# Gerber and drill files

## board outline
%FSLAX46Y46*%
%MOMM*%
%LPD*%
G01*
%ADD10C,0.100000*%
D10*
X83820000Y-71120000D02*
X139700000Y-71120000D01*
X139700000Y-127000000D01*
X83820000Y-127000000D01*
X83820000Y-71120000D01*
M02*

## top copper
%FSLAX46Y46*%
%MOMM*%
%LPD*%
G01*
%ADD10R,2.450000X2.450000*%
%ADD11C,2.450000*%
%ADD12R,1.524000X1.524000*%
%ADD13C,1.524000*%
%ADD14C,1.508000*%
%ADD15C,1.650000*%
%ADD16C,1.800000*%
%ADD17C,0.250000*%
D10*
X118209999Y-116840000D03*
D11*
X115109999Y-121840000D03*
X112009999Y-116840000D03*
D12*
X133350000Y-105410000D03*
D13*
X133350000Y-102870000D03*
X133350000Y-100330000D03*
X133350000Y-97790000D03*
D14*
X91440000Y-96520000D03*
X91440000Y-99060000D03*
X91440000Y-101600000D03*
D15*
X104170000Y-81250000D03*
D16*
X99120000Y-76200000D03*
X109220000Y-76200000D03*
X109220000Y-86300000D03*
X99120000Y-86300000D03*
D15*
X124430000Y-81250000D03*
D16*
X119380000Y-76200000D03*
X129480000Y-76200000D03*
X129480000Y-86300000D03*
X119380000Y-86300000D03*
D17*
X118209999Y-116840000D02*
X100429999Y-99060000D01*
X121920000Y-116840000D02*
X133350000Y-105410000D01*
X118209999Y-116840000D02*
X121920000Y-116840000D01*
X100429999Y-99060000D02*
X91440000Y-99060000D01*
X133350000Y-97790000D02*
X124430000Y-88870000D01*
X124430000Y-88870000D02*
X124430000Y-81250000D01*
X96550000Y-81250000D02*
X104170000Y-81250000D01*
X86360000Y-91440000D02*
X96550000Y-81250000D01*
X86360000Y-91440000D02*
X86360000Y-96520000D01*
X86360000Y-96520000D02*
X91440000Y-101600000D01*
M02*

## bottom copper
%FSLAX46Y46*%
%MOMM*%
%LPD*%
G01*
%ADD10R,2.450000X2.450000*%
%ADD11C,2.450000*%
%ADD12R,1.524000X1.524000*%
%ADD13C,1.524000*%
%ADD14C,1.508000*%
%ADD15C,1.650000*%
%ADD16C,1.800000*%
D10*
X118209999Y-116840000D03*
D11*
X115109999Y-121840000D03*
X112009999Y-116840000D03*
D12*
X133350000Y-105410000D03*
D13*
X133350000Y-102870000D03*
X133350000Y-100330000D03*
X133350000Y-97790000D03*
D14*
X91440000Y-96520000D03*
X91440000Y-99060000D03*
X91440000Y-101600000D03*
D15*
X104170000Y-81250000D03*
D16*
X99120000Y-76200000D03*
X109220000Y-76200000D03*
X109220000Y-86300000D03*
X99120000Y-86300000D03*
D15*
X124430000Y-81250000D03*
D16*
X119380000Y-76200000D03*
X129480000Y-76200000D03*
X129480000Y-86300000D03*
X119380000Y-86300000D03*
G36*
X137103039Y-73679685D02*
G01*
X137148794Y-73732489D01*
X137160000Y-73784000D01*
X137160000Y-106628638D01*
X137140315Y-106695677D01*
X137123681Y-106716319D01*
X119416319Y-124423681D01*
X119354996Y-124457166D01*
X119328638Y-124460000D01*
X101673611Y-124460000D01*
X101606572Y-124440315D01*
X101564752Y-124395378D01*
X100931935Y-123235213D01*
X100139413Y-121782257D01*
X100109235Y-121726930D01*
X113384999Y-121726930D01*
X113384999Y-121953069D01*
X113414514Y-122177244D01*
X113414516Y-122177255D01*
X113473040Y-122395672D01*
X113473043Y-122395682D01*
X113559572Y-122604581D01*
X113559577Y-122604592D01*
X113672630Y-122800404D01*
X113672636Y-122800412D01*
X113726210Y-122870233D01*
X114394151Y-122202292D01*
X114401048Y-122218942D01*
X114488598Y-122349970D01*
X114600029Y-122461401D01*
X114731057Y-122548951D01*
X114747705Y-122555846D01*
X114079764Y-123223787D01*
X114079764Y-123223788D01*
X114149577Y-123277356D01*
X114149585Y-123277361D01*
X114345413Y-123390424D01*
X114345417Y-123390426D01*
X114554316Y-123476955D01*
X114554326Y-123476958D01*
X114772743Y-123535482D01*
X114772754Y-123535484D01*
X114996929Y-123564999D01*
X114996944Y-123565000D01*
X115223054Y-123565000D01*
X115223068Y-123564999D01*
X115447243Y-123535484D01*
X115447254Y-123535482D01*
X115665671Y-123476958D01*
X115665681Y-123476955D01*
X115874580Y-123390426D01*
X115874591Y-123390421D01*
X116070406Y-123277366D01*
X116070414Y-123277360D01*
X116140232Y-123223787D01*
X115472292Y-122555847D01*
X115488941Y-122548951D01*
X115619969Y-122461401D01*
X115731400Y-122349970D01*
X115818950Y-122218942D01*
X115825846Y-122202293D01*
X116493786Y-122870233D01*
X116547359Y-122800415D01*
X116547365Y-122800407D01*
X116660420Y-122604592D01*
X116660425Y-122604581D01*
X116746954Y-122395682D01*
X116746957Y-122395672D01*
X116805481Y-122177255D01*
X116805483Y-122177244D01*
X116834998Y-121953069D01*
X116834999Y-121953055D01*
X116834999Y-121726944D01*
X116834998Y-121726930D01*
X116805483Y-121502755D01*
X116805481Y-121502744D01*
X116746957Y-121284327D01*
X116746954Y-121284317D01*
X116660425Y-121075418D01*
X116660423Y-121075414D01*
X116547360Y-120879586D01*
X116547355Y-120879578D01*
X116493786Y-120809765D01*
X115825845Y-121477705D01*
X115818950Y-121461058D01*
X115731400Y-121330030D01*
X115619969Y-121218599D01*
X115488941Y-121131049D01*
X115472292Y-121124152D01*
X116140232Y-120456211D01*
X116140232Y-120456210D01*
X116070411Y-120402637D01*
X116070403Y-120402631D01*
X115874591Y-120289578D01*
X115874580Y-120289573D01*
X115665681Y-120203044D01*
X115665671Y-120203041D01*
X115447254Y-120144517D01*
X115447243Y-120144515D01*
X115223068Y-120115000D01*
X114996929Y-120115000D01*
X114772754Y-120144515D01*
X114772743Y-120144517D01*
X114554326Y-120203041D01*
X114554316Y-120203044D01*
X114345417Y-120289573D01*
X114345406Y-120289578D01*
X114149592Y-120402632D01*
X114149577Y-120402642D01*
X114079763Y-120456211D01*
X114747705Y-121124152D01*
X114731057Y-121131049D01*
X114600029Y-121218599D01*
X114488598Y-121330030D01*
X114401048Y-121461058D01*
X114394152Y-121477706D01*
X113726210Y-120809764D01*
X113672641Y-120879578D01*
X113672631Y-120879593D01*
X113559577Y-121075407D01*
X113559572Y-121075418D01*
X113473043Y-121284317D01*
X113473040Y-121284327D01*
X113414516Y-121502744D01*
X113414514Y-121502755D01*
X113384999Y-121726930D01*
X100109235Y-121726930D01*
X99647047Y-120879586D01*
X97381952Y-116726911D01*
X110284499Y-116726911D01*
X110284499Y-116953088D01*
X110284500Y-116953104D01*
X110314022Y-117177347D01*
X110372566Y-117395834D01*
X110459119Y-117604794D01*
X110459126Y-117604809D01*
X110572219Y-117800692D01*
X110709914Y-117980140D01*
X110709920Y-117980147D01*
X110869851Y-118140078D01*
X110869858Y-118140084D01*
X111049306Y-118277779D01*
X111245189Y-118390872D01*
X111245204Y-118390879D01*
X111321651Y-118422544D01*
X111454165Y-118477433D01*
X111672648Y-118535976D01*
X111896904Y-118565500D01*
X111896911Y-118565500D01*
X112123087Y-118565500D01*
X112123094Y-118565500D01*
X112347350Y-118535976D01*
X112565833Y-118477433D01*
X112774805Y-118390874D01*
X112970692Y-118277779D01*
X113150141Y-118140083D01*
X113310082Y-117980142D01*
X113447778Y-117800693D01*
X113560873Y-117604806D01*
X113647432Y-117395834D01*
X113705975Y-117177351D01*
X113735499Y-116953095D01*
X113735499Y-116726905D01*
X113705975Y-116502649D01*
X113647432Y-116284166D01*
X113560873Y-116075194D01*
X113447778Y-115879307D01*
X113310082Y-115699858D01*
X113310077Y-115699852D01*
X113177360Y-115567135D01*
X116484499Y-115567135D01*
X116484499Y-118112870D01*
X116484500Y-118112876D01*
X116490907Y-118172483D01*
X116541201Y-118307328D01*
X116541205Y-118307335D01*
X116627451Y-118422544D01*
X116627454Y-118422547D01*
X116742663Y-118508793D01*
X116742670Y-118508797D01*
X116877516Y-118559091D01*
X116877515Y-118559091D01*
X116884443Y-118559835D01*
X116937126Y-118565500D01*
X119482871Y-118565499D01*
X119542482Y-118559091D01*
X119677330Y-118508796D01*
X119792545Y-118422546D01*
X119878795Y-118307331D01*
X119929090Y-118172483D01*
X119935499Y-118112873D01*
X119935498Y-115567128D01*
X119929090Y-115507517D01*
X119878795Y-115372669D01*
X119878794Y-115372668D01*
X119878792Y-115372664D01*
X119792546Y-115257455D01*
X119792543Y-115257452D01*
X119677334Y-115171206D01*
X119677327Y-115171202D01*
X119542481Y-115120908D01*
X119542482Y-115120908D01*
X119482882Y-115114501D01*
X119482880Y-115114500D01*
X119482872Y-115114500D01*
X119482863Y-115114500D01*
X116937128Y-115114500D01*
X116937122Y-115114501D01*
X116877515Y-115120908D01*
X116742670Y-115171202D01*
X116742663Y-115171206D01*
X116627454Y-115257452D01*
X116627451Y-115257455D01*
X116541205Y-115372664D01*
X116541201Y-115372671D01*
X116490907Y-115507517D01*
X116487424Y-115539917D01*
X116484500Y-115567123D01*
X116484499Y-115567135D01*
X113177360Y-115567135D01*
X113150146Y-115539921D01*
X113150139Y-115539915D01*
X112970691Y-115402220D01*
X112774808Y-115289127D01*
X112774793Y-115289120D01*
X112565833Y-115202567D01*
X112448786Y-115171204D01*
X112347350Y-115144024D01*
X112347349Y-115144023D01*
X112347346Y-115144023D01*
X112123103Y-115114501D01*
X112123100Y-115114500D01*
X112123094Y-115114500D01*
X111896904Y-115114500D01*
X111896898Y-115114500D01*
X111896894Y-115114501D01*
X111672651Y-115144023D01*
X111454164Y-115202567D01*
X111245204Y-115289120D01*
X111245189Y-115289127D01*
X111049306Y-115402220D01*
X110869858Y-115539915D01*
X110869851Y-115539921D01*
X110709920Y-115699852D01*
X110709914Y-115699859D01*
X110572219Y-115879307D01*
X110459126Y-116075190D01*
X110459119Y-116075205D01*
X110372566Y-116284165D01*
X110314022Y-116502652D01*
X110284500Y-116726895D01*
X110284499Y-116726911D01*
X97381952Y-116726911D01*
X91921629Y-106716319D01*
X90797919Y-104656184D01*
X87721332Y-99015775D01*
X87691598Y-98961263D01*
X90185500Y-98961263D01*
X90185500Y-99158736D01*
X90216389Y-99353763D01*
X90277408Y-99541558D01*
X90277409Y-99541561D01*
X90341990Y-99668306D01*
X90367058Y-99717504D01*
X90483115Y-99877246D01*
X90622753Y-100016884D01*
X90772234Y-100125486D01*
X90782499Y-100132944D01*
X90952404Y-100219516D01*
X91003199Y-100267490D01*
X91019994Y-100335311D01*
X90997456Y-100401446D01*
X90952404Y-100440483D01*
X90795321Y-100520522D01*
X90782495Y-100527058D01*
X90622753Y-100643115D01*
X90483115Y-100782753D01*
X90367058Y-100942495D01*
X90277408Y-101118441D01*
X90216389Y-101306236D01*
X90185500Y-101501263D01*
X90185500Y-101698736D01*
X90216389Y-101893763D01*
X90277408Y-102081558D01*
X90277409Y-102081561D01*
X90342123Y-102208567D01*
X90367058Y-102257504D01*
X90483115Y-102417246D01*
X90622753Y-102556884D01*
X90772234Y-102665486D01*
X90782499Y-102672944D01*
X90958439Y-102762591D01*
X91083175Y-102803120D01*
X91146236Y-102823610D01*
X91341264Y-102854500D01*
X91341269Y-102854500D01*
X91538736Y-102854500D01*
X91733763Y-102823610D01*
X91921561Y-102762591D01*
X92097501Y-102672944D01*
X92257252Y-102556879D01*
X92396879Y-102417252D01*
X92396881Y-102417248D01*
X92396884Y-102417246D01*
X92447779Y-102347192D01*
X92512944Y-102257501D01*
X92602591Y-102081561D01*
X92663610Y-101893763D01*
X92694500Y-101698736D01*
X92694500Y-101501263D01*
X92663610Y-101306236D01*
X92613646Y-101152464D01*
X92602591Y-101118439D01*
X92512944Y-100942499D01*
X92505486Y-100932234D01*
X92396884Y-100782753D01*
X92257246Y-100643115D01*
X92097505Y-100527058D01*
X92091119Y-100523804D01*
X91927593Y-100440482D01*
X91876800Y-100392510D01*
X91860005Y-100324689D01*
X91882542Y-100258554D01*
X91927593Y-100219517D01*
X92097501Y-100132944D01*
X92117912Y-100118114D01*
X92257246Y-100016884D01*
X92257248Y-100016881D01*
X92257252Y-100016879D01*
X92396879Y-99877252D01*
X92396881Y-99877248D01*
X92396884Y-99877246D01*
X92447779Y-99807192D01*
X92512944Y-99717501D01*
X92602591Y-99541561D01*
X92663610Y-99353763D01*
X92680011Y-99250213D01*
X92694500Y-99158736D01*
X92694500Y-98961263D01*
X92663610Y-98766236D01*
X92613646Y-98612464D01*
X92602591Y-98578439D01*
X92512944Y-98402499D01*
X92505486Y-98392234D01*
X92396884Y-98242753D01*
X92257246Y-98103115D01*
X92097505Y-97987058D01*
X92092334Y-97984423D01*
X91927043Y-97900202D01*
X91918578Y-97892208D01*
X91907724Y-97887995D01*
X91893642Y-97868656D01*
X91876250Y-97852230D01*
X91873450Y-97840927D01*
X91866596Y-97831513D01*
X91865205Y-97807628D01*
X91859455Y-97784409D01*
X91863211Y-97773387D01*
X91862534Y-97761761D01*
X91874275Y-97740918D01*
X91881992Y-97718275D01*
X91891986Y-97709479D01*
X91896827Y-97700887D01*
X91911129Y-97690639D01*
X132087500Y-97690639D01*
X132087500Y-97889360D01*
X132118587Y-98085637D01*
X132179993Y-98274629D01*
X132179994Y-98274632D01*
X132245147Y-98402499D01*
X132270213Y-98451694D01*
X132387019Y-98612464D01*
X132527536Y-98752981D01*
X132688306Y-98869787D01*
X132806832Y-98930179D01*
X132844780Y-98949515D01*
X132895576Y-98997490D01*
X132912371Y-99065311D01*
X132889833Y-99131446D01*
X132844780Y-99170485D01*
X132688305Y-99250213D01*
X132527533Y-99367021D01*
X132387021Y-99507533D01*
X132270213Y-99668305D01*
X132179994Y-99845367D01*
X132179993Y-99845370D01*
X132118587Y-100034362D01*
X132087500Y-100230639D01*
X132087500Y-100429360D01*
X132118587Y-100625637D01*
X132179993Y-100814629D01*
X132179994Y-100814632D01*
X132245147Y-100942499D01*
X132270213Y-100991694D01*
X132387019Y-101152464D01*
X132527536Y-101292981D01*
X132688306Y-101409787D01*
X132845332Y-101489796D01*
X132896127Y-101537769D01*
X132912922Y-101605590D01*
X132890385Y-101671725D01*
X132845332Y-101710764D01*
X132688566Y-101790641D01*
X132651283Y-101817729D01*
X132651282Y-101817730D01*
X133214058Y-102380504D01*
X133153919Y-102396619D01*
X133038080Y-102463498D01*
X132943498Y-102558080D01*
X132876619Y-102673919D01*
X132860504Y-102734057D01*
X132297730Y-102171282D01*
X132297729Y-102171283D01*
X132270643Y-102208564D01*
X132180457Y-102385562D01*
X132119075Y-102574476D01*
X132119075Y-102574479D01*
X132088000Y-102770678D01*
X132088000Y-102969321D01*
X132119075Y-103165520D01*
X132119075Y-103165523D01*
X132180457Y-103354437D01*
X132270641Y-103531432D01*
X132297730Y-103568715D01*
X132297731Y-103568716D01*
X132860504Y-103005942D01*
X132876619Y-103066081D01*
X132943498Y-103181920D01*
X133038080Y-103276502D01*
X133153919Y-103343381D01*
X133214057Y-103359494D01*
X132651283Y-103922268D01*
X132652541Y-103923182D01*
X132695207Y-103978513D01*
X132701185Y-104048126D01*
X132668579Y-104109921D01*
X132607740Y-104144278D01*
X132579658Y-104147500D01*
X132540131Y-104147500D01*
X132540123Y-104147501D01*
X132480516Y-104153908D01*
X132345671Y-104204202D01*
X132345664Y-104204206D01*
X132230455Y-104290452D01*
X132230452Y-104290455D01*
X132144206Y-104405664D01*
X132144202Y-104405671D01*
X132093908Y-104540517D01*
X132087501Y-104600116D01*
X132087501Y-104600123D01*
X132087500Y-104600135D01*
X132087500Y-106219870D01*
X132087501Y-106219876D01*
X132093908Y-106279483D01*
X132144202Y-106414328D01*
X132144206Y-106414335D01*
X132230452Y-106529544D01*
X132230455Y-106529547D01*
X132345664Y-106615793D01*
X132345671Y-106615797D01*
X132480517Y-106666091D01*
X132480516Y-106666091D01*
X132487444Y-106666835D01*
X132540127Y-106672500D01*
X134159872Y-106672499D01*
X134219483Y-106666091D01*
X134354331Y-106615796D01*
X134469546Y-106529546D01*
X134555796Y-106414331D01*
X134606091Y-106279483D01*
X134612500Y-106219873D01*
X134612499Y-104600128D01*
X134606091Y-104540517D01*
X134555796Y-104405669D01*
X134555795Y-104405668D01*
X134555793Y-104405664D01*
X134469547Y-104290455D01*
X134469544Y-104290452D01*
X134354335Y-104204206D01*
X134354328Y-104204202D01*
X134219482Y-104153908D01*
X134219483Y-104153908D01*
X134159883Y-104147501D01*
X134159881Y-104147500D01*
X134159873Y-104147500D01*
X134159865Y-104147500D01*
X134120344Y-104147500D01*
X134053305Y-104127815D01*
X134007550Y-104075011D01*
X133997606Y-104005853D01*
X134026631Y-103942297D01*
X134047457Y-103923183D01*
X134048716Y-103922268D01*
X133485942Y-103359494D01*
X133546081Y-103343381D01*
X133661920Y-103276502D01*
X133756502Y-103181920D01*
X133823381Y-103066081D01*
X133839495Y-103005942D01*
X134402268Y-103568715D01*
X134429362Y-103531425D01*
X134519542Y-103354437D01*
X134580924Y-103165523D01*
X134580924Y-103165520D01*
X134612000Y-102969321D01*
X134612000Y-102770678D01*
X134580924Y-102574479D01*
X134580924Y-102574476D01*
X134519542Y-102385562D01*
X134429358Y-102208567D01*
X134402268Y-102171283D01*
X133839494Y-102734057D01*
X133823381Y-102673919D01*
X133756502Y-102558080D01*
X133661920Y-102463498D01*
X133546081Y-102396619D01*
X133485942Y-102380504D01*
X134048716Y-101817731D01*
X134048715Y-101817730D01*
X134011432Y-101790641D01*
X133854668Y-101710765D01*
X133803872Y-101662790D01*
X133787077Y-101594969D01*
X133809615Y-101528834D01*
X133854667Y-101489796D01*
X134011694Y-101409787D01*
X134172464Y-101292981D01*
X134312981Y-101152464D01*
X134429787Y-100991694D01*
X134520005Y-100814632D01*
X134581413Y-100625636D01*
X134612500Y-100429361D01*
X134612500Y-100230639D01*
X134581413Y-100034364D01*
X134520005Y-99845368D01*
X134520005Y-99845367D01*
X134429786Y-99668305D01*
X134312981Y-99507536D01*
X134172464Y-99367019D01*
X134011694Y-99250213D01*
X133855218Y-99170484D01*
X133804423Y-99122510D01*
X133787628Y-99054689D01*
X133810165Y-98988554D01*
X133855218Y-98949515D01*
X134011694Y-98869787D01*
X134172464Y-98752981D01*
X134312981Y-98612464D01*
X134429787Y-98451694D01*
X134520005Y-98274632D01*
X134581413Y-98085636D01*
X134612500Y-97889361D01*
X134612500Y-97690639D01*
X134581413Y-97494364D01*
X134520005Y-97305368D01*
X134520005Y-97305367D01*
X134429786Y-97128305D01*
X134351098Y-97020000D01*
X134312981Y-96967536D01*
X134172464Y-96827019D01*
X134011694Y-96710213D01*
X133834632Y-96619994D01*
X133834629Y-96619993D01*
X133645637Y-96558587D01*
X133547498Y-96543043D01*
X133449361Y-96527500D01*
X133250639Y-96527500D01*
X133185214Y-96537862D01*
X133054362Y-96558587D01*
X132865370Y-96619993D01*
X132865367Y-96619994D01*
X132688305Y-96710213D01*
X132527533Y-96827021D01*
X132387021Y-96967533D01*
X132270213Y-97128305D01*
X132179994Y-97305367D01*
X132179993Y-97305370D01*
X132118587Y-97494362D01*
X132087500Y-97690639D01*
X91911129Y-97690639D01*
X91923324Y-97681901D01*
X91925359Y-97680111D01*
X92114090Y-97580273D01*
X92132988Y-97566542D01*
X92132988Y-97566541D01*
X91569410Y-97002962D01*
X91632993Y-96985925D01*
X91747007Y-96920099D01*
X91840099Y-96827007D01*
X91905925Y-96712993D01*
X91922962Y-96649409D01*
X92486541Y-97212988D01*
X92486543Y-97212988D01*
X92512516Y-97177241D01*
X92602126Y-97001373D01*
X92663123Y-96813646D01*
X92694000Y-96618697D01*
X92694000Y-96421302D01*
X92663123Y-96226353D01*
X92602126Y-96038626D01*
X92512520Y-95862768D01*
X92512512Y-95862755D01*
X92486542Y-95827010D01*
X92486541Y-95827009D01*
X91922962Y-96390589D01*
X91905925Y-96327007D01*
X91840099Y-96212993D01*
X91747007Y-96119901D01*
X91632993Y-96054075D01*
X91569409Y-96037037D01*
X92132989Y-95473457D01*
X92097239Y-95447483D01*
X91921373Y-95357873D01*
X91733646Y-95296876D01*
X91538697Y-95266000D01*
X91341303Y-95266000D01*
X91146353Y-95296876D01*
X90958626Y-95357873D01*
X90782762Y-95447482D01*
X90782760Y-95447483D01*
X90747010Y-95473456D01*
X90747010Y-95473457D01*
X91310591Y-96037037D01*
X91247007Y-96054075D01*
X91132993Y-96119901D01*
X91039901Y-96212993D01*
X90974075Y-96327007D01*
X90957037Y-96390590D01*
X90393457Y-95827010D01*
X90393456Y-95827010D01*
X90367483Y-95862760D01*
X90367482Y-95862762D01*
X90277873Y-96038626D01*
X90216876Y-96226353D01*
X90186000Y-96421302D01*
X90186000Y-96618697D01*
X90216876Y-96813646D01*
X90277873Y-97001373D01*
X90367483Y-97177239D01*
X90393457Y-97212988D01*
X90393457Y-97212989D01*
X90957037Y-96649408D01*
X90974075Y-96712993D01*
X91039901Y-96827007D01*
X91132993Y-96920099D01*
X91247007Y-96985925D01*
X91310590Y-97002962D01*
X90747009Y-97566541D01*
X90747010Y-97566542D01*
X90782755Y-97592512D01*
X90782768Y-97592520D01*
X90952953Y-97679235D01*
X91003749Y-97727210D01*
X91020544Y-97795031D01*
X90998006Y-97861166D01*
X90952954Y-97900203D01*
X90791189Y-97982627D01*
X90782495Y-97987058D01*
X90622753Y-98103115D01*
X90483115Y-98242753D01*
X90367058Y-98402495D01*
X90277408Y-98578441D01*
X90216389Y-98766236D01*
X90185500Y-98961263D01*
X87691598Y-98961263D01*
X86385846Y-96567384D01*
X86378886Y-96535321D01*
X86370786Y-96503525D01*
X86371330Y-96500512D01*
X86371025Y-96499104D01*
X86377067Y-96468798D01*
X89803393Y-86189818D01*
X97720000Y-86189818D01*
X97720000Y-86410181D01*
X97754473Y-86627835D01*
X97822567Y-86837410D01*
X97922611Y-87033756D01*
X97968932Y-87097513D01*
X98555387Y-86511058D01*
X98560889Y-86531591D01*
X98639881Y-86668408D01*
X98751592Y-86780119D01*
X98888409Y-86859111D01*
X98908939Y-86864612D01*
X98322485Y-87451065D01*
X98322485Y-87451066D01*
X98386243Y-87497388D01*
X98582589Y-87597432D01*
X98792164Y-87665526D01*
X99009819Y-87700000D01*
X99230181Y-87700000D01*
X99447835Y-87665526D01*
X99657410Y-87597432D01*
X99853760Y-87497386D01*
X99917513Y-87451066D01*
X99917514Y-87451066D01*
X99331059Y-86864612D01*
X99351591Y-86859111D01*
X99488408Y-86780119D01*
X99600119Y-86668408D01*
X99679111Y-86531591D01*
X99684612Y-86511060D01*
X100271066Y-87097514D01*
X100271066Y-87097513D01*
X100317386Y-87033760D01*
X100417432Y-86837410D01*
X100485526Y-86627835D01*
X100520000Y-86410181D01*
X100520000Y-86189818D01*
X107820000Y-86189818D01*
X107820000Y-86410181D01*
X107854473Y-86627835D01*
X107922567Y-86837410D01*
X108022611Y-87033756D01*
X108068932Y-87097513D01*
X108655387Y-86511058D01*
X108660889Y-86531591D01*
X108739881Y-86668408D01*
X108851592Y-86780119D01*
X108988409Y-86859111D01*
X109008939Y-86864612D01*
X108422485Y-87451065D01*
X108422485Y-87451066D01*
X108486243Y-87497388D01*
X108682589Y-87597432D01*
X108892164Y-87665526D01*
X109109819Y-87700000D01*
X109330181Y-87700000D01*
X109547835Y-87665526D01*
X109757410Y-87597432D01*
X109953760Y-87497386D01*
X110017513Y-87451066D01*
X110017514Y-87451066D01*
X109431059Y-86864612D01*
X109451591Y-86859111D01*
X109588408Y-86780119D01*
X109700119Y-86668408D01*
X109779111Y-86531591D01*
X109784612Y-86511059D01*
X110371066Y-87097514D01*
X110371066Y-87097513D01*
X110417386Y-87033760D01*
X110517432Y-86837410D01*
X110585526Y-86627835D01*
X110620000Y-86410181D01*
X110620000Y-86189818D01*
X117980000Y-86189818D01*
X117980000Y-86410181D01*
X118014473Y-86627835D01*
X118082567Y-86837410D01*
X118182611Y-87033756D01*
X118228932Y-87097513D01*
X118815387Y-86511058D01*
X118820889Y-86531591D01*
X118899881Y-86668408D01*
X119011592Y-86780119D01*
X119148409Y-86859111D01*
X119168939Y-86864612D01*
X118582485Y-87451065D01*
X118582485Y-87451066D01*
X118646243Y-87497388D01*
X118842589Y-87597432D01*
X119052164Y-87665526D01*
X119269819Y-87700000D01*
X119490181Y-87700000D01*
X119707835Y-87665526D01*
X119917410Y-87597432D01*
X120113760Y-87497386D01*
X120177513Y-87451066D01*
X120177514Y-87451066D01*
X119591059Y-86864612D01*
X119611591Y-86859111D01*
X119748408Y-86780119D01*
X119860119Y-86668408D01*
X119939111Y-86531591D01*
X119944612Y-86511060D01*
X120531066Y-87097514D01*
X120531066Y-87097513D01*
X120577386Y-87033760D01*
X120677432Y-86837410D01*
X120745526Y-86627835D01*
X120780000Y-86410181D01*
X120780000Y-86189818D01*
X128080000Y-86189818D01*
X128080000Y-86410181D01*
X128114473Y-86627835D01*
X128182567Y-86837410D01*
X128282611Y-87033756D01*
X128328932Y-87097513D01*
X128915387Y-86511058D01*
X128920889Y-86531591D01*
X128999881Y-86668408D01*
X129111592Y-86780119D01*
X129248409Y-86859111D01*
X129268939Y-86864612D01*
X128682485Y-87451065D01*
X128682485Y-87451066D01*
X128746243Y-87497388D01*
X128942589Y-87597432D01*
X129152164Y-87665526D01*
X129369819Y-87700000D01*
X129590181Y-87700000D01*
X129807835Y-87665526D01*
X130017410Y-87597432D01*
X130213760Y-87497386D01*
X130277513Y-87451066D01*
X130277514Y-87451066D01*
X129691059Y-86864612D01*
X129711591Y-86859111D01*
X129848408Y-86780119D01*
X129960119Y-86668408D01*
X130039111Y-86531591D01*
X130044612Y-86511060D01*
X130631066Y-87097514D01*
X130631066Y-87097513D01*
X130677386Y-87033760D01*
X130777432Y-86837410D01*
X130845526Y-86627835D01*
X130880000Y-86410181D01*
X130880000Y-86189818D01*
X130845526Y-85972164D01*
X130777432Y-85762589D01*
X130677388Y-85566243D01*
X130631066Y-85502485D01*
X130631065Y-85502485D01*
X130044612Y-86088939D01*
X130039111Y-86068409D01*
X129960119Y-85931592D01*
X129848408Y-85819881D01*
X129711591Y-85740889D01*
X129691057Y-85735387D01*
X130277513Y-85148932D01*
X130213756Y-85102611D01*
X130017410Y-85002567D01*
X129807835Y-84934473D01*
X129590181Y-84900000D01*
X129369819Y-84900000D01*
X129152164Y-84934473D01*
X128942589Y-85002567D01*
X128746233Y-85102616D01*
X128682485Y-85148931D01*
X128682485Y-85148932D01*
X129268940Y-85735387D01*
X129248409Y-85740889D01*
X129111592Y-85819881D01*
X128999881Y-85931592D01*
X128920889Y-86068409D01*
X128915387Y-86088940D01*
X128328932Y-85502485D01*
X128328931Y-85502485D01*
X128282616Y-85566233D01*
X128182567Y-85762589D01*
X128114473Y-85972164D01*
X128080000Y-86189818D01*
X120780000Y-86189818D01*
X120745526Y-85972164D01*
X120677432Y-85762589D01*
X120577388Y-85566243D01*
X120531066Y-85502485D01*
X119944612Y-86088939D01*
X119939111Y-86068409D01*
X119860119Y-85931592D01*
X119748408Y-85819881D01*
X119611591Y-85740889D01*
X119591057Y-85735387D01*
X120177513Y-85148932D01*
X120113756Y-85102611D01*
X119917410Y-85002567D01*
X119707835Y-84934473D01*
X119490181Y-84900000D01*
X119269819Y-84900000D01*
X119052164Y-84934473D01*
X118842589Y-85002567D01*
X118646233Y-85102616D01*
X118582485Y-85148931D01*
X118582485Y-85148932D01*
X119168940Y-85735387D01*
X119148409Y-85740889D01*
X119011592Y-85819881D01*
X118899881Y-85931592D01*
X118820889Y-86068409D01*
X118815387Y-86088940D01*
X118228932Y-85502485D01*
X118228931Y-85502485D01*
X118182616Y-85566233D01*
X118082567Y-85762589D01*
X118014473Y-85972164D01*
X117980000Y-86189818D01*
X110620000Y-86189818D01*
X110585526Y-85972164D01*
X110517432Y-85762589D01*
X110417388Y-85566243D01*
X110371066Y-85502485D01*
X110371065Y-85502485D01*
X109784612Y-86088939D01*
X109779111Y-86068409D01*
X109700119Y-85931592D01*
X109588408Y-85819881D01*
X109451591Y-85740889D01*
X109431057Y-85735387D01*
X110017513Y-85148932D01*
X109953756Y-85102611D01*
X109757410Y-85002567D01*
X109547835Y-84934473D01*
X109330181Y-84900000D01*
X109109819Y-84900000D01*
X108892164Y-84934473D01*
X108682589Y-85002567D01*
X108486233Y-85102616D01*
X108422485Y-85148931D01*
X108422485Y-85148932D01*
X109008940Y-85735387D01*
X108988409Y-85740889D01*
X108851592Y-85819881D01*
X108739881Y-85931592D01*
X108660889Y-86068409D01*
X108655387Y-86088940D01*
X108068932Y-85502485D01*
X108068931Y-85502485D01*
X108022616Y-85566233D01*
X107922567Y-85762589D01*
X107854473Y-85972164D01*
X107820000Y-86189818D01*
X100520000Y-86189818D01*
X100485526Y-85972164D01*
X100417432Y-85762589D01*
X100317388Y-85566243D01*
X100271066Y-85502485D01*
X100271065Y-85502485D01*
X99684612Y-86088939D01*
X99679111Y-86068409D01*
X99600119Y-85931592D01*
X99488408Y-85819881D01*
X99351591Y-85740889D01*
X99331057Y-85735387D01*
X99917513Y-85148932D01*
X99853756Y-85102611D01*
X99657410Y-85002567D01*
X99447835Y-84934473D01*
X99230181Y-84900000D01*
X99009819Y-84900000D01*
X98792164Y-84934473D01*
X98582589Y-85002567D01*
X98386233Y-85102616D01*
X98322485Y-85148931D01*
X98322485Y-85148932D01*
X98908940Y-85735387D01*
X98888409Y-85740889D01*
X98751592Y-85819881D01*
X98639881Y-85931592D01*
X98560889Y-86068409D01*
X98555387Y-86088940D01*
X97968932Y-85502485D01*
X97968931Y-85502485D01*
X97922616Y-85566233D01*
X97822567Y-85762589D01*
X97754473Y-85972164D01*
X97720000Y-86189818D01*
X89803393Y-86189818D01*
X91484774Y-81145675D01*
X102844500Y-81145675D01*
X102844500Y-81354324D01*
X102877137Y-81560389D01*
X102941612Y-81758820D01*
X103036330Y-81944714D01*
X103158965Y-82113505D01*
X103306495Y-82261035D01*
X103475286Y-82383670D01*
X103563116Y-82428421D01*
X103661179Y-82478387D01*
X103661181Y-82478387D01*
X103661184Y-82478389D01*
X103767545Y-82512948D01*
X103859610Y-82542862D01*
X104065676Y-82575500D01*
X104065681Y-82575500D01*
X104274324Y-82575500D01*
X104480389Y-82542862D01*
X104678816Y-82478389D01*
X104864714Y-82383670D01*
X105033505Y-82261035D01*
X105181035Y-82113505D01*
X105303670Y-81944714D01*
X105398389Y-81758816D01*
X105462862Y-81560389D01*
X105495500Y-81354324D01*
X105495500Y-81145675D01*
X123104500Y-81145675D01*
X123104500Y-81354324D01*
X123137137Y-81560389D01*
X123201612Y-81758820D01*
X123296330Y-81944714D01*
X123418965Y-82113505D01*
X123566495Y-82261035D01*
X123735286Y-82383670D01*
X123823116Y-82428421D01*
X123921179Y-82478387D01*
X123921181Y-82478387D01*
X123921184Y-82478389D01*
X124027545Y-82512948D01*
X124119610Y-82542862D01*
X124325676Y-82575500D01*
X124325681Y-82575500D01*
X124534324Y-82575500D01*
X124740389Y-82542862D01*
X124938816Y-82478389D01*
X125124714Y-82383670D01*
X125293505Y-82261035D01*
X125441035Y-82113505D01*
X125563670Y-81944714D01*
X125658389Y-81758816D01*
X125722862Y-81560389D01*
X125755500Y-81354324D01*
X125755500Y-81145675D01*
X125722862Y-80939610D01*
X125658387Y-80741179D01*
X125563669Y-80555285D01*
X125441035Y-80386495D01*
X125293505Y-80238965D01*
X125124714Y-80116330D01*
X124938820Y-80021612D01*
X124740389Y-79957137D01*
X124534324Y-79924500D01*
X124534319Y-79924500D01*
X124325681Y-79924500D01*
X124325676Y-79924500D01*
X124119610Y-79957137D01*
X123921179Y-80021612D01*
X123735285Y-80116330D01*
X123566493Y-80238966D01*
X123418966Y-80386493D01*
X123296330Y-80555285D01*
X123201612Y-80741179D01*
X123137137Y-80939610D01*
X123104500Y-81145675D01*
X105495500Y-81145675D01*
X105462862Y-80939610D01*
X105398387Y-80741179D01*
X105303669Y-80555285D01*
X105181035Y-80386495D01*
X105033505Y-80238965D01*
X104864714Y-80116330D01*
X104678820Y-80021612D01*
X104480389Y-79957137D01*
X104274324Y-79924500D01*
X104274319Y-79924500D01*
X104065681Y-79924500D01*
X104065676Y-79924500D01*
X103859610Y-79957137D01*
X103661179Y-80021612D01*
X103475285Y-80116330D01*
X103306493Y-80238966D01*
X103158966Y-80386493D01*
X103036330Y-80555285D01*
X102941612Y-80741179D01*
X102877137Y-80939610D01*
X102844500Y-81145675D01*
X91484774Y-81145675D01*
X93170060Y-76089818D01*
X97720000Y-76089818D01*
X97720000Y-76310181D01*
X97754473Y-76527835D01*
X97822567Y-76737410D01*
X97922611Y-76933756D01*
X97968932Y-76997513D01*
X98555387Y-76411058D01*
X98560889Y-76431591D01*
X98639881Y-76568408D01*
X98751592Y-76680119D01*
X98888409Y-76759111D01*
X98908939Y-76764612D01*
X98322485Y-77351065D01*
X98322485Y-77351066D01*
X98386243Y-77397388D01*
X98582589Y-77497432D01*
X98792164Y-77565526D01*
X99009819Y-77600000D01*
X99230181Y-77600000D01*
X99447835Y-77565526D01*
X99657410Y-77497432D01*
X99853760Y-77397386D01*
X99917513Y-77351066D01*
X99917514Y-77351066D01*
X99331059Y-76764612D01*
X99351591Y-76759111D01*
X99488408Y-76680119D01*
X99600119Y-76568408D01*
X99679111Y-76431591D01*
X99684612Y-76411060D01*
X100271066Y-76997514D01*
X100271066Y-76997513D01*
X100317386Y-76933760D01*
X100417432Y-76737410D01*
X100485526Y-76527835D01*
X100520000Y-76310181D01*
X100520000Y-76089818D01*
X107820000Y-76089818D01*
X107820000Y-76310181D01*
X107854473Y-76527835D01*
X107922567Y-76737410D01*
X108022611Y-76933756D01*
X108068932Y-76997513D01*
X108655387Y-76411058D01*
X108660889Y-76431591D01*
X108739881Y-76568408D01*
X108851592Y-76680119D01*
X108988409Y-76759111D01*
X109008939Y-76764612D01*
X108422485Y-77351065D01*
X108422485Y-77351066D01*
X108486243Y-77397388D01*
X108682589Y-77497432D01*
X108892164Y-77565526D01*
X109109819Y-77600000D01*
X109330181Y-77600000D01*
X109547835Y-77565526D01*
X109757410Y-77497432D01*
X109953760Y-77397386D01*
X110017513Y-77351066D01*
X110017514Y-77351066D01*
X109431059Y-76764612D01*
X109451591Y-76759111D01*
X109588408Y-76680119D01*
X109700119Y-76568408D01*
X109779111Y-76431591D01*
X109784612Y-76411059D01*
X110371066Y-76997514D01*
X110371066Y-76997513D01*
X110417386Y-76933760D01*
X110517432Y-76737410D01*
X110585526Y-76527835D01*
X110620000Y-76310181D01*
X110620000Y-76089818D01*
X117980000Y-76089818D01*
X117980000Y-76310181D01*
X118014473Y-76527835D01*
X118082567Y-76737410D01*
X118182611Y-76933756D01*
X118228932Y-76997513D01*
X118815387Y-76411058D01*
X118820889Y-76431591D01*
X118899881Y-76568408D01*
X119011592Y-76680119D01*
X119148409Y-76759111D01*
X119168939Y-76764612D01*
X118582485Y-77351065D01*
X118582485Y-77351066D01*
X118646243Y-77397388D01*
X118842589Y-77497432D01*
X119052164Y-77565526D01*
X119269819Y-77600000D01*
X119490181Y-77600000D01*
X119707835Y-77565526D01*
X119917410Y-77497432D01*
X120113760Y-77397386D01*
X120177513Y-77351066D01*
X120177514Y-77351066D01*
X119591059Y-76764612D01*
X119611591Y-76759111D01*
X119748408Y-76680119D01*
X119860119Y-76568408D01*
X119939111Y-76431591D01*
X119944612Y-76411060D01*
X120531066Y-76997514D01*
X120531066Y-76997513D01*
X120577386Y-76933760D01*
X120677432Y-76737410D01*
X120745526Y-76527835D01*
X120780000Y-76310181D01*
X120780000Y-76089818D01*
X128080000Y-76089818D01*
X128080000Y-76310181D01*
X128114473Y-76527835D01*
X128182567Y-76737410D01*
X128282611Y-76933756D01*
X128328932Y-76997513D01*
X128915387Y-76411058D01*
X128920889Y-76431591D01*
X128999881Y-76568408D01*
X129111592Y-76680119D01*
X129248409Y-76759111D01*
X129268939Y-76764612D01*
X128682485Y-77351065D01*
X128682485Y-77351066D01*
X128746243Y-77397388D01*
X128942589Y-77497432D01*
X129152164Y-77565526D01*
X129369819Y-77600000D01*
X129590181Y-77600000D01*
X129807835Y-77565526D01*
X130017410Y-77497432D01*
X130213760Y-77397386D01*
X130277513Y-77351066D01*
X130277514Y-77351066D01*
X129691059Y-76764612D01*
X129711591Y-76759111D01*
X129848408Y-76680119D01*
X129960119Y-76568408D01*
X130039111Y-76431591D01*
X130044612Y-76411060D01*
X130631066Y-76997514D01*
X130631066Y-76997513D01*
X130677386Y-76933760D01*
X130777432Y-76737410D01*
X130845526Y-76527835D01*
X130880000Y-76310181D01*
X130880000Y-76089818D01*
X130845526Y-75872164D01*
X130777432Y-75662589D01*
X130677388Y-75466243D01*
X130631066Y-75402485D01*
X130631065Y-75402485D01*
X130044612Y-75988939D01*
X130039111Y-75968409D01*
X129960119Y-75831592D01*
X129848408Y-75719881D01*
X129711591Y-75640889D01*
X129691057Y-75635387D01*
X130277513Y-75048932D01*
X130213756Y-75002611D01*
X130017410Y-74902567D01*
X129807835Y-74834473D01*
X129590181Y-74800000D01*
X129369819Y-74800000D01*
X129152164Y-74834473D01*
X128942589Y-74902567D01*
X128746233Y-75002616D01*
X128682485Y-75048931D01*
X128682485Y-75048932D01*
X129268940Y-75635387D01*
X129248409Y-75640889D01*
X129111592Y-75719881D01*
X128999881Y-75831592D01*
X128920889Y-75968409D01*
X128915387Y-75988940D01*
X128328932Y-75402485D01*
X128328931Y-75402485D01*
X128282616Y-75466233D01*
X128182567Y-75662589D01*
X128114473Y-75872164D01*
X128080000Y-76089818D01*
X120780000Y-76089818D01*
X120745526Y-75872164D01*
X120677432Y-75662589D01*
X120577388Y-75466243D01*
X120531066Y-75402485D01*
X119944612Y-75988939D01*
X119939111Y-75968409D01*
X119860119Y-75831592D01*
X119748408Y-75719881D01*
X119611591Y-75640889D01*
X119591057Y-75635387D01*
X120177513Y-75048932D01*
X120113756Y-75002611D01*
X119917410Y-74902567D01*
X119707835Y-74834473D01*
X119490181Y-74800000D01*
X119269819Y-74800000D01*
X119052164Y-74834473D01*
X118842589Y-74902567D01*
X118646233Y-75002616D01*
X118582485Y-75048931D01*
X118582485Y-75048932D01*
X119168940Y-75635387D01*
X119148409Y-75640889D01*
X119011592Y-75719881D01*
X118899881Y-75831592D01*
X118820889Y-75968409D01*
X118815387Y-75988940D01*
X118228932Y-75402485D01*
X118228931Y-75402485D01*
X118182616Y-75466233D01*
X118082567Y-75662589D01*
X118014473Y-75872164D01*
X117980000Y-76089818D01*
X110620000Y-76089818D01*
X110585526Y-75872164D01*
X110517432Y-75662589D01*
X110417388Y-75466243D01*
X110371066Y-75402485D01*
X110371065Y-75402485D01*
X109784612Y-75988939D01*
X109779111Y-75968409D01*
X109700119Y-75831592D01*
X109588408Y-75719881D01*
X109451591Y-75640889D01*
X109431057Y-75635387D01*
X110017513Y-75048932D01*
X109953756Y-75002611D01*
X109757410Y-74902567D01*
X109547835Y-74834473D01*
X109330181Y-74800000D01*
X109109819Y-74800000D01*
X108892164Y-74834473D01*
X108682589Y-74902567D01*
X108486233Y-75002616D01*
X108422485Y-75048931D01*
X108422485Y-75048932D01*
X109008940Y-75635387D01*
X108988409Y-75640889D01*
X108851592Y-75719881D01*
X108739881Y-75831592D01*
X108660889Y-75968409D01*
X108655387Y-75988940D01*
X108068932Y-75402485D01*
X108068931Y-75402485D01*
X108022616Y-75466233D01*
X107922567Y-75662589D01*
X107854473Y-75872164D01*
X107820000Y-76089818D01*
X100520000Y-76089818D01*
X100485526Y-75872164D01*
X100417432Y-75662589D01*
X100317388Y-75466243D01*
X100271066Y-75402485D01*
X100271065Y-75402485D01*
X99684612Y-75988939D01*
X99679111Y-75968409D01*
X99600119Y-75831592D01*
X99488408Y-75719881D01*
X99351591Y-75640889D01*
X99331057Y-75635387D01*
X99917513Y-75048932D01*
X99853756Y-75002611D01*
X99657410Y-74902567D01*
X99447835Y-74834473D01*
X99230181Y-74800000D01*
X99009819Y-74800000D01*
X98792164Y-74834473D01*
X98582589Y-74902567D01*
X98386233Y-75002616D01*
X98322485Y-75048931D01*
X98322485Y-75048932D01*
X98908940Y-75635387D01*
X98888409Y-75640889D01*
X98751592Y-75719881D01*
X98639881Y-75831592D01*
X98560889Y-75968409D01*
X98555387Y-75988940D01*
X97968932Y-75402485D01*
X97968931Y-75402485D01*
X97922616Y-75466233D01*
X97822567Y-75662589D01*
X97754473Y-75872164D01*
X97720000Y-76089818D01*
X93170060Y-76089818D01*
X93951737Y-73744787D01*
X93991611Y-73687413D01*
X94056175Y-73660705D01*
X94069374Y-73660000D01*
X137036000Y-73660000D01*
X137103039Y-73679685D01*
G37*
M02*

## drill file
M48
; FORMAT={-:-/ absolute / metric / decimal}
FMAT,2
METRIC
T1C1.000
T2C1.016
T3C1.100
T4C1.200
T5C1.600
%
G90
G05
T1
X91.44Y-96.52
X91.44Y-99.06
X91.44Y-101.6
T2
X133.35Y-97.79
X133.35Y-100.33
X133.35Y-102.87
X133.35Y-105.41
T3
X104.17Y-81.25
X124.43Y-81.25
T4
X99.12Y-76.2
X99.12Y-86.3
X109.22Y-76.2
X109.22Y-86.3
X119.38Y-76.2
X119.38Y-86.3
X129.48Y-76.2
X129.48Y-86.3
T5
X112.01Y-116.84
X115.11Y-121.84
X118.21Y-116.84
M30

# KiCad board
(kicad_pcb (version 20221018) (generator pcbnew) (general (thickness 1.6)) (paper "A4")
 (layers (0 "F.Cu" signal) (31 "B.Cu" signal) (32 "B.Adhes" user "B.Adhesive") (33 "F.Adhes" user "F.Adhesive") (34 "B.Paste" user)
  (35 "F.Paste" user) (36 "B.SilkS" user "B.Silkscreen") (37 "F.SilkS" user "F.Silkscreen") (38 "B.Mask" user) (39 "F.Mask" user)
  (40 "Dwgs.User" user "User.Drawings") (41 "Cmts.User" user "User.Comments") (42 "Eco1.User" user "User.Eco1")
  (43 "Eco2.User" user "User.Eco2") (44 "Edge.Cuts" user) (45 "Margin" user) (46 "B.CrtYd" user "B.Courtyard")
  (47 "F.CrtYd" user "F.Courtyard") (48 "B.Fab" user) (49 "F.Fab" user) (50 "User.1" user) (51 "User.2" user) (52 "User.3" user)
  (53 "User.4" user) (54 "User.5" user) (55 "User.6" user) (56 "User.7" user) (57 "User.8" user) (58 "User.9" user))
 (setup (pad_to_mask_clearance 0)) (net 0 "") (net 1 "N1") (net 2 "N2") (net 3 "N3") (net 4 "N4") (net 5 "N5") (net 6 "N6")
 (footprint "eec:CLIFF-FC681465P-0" (layer "F.Cu") (at 111.76 116.84)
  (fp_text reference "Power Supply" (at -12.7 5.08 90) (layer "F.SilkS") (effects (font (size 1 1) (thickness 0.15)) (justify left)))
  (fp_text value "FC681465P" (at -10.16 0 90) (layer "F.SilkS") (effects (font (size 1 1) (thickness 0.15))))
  (pad "1" thru_hole rect (at 6.449999 0) (size 2.45 2.45) (drill 1.6) (layers "*.Cu") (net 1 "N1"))
  (pad "2" thru_hole circle (at 3.349999 5) (size 2.45 2.45) (drill 1.6) (layers "*.Cu") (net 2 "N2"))
  (pad "3" thru_hole circle (at 0.249999 0) (size 2.45 2.45) (drill 1.6) (layers "*.Cu") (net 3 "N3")))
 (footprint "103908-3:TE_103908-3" (layer "F.Cu") (at 133.35 101.6 90)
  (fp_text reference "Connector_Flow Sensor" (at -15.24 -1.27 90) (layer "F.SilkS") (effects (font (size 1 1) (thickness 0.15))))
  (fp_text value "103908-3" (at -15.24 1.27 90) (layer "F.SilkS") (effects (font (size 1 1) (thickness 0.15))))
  (pad "1" thru_hole rect (at -3.81 0 90) (size 1.524 1.524) (drill 1.016) (layers "*.Cu" "*.Mask") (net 1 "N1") (solder_mask_margin 0.102))
  (pad "2" thru_hole circle (at -1.27 0 90) (size 1.524 1.524) (drill 1.016) (layers "*.Cu" "*.Mask") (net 2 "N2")
   (solder_mask_margin 0.102))
  (pad "3" thru_hole circle (at 1.27 0 90) (size 1.524 1.524) (drill 1.016) (layers "*.Cu" "*.Mask") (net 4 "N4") (solder_mask_margin 0.102))
  (pad "4" thru_hole circle (at 3.81 0 90) (size 1.524 1.524) (drill 1.016) (layers "*.Cu" "*.Mask") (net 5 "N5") (solder_mask_margin 0.102)))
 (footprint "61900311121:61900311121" (layer "F.Cu") (at 91.44 99.06 90)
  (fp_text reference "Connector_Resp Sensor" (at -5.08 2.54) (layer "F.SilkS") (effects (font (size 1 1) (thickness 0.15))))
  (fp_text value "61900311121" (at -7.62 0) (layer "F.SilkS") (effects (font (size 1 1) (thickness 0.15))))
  (pad "1" thru_hole circle (at 2.54 0 90) (size 1.508 1.508) (drill 1) (layers "*.Cu" "*.Mask") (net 2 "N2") (solder_mask_margin 0.102))
  (pad "2" thru_hole circle (at 0 0 90) (size 1.508 1.508) (drill 1) (layers "*.Cu" "*.Mask") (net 1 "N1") (solder_mask_margin 0.102))
  (pad "3" thru_hole circle (at -2.54 0 90) (size 1.508 1.508) (drill 1) (layers "*.Cu" "*.Mask") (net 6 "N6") (solder_mask_margin 0.102)))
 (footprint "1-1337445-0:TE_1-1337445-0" (layer "F.Cu") (at 104.17 81.25)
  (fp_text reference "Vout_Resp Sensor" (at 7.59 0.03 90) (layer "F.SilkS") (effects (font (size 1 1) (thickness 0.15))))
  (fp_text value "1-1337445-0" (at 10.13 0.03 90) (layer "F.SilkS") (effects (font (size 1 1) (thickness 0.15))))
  (pad "1" thru_hole circle (at 0 0) (size 1.65 1.65) (drill 1.1) (layers "*.Cu" "*.Mask") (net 6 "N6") (solder_mask_margin 0.102))
  (pad "2" thru_hole circle (at -5.05 -5.05) (size 1.8 1.8) (drill 1.2) (layers "*.Cu" "*.Mask") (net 2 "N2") (solder_mask_margin 0.102))
  (pad "3" thru_hole circle (at 5.05 -5.05) (size 1.8 1.8) (drill 1.2) (layers "*.Cu" "*.Mask") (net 2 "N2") (solder_mask_margin 0.102))
  (pad "4" thru_hole circle (at 5.05 5.05) (size 1.8 1.8) (drill 1.2) (layers "*.Cu" "*.Mask") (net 2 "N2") (solder_mask_margin 0.102))
  (pad "5" thru_hole circle (at -5.05 5.05) (size 1.8 1.8) (drill 1.2) (layers "*.Cu" "*.Mask") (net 2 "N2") (solder_mask_margin 0.102)))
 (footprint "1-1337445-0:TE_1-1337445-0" (layer "F.Cu") (at 124.43 81.25)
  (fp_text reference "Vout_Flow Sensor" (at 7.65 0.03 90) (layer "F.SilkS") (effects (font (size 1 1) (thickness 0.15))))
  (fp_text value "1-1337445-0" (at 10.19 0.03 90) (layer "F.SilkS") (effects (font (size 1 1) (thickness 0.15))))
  (pad "1" thru_hole circle (at 0 0) (size 1.65 1.65) (drill 1.1) (layers "*.Cu" "*.Mask") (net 5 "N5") (solder_mask_margin 0.102))
  (pad "2" thru_hole circle (at -5.05 -5.05) (size 1.8 1.8) (drill 1.2) (layers "*.Cu" "*.Mask") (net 2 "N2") (solder_mask_margin 0.102))
  (pad "3" thru_hole circle (at 5.05 -5.05) (size 1.8 1.8) (drill 1.2) (layers "*.Cu" "*.Mask") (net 2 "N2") (solder_mask_margin 0.102))
  (pad "4" thru_hole circle (at 5.05 5.05) (size 1.8 1.8) (drill 1.2) (layers "*.Cu" "*.Mask") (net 2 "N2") (solder_mask_margin 0.102))
  (pad "5" thru_hole circle (at -5.05 5.05) (size 1.8 1.8) (drill 1.2) (layers "*.Cu" "*.Mask") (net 2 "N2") (solder_mask_margin 0.102)))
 (gr_rect (start 83.82 71.12) (end 139.7 127) (stroke (width 0.1) (type default)) (fill none) (layer "Edge.Cuts"))
 (segment (start 118.209999 116.84) (end 100.429999 99.06) (width 0.25) (layer "F.Cu") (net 1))
 (segment (start 121.92 116.84) (end 133.35 105.41) (width 0.25) (layer "F.Cu") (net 1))
 (segment (start 118.209999 116.84) (end 121.92 116.84) (width 0.25) (layer "F.Cu") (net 1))
 (segment (start 100.429999 99.06) (end 91.44 99.06) (width 0.25) (layer "F.Cu") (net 1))
 (segment (start 133.35 97.79) (end 124.43 88.87) (width 0.25) (layer "F.Cu") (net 5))
 (segment (start 124.43 88.87) (end 124.43 81.25) (width 0.25) (layer "F.Cu") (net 5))
 (segment (start 96.55 81.25) (end 104.17 81.25) (width 0.25) (layer "F.Cu") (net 6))
 (segment (start 86.36 91.44) (end 96.55 81.25) (width 0.25) (layer "F.Cu") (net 6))
 (segment (start 86.36 91.44) (end 86.36 96.52) (width 0.25) (layer "F.Cu") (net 6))
 (segment (start 86.36 96.52) (end 91.44 101.6) (width 0.25) (layer "F.Cu") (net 6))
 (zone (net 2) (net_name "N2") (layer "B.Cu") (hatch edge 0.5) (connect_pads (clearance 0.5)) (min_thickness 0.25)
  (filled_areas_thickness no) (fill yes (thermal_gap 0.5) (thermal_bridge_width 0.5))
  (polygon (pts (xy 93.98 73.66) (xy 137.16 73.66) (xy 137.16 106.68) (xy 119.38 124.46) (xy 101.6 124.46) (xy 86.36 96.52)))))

